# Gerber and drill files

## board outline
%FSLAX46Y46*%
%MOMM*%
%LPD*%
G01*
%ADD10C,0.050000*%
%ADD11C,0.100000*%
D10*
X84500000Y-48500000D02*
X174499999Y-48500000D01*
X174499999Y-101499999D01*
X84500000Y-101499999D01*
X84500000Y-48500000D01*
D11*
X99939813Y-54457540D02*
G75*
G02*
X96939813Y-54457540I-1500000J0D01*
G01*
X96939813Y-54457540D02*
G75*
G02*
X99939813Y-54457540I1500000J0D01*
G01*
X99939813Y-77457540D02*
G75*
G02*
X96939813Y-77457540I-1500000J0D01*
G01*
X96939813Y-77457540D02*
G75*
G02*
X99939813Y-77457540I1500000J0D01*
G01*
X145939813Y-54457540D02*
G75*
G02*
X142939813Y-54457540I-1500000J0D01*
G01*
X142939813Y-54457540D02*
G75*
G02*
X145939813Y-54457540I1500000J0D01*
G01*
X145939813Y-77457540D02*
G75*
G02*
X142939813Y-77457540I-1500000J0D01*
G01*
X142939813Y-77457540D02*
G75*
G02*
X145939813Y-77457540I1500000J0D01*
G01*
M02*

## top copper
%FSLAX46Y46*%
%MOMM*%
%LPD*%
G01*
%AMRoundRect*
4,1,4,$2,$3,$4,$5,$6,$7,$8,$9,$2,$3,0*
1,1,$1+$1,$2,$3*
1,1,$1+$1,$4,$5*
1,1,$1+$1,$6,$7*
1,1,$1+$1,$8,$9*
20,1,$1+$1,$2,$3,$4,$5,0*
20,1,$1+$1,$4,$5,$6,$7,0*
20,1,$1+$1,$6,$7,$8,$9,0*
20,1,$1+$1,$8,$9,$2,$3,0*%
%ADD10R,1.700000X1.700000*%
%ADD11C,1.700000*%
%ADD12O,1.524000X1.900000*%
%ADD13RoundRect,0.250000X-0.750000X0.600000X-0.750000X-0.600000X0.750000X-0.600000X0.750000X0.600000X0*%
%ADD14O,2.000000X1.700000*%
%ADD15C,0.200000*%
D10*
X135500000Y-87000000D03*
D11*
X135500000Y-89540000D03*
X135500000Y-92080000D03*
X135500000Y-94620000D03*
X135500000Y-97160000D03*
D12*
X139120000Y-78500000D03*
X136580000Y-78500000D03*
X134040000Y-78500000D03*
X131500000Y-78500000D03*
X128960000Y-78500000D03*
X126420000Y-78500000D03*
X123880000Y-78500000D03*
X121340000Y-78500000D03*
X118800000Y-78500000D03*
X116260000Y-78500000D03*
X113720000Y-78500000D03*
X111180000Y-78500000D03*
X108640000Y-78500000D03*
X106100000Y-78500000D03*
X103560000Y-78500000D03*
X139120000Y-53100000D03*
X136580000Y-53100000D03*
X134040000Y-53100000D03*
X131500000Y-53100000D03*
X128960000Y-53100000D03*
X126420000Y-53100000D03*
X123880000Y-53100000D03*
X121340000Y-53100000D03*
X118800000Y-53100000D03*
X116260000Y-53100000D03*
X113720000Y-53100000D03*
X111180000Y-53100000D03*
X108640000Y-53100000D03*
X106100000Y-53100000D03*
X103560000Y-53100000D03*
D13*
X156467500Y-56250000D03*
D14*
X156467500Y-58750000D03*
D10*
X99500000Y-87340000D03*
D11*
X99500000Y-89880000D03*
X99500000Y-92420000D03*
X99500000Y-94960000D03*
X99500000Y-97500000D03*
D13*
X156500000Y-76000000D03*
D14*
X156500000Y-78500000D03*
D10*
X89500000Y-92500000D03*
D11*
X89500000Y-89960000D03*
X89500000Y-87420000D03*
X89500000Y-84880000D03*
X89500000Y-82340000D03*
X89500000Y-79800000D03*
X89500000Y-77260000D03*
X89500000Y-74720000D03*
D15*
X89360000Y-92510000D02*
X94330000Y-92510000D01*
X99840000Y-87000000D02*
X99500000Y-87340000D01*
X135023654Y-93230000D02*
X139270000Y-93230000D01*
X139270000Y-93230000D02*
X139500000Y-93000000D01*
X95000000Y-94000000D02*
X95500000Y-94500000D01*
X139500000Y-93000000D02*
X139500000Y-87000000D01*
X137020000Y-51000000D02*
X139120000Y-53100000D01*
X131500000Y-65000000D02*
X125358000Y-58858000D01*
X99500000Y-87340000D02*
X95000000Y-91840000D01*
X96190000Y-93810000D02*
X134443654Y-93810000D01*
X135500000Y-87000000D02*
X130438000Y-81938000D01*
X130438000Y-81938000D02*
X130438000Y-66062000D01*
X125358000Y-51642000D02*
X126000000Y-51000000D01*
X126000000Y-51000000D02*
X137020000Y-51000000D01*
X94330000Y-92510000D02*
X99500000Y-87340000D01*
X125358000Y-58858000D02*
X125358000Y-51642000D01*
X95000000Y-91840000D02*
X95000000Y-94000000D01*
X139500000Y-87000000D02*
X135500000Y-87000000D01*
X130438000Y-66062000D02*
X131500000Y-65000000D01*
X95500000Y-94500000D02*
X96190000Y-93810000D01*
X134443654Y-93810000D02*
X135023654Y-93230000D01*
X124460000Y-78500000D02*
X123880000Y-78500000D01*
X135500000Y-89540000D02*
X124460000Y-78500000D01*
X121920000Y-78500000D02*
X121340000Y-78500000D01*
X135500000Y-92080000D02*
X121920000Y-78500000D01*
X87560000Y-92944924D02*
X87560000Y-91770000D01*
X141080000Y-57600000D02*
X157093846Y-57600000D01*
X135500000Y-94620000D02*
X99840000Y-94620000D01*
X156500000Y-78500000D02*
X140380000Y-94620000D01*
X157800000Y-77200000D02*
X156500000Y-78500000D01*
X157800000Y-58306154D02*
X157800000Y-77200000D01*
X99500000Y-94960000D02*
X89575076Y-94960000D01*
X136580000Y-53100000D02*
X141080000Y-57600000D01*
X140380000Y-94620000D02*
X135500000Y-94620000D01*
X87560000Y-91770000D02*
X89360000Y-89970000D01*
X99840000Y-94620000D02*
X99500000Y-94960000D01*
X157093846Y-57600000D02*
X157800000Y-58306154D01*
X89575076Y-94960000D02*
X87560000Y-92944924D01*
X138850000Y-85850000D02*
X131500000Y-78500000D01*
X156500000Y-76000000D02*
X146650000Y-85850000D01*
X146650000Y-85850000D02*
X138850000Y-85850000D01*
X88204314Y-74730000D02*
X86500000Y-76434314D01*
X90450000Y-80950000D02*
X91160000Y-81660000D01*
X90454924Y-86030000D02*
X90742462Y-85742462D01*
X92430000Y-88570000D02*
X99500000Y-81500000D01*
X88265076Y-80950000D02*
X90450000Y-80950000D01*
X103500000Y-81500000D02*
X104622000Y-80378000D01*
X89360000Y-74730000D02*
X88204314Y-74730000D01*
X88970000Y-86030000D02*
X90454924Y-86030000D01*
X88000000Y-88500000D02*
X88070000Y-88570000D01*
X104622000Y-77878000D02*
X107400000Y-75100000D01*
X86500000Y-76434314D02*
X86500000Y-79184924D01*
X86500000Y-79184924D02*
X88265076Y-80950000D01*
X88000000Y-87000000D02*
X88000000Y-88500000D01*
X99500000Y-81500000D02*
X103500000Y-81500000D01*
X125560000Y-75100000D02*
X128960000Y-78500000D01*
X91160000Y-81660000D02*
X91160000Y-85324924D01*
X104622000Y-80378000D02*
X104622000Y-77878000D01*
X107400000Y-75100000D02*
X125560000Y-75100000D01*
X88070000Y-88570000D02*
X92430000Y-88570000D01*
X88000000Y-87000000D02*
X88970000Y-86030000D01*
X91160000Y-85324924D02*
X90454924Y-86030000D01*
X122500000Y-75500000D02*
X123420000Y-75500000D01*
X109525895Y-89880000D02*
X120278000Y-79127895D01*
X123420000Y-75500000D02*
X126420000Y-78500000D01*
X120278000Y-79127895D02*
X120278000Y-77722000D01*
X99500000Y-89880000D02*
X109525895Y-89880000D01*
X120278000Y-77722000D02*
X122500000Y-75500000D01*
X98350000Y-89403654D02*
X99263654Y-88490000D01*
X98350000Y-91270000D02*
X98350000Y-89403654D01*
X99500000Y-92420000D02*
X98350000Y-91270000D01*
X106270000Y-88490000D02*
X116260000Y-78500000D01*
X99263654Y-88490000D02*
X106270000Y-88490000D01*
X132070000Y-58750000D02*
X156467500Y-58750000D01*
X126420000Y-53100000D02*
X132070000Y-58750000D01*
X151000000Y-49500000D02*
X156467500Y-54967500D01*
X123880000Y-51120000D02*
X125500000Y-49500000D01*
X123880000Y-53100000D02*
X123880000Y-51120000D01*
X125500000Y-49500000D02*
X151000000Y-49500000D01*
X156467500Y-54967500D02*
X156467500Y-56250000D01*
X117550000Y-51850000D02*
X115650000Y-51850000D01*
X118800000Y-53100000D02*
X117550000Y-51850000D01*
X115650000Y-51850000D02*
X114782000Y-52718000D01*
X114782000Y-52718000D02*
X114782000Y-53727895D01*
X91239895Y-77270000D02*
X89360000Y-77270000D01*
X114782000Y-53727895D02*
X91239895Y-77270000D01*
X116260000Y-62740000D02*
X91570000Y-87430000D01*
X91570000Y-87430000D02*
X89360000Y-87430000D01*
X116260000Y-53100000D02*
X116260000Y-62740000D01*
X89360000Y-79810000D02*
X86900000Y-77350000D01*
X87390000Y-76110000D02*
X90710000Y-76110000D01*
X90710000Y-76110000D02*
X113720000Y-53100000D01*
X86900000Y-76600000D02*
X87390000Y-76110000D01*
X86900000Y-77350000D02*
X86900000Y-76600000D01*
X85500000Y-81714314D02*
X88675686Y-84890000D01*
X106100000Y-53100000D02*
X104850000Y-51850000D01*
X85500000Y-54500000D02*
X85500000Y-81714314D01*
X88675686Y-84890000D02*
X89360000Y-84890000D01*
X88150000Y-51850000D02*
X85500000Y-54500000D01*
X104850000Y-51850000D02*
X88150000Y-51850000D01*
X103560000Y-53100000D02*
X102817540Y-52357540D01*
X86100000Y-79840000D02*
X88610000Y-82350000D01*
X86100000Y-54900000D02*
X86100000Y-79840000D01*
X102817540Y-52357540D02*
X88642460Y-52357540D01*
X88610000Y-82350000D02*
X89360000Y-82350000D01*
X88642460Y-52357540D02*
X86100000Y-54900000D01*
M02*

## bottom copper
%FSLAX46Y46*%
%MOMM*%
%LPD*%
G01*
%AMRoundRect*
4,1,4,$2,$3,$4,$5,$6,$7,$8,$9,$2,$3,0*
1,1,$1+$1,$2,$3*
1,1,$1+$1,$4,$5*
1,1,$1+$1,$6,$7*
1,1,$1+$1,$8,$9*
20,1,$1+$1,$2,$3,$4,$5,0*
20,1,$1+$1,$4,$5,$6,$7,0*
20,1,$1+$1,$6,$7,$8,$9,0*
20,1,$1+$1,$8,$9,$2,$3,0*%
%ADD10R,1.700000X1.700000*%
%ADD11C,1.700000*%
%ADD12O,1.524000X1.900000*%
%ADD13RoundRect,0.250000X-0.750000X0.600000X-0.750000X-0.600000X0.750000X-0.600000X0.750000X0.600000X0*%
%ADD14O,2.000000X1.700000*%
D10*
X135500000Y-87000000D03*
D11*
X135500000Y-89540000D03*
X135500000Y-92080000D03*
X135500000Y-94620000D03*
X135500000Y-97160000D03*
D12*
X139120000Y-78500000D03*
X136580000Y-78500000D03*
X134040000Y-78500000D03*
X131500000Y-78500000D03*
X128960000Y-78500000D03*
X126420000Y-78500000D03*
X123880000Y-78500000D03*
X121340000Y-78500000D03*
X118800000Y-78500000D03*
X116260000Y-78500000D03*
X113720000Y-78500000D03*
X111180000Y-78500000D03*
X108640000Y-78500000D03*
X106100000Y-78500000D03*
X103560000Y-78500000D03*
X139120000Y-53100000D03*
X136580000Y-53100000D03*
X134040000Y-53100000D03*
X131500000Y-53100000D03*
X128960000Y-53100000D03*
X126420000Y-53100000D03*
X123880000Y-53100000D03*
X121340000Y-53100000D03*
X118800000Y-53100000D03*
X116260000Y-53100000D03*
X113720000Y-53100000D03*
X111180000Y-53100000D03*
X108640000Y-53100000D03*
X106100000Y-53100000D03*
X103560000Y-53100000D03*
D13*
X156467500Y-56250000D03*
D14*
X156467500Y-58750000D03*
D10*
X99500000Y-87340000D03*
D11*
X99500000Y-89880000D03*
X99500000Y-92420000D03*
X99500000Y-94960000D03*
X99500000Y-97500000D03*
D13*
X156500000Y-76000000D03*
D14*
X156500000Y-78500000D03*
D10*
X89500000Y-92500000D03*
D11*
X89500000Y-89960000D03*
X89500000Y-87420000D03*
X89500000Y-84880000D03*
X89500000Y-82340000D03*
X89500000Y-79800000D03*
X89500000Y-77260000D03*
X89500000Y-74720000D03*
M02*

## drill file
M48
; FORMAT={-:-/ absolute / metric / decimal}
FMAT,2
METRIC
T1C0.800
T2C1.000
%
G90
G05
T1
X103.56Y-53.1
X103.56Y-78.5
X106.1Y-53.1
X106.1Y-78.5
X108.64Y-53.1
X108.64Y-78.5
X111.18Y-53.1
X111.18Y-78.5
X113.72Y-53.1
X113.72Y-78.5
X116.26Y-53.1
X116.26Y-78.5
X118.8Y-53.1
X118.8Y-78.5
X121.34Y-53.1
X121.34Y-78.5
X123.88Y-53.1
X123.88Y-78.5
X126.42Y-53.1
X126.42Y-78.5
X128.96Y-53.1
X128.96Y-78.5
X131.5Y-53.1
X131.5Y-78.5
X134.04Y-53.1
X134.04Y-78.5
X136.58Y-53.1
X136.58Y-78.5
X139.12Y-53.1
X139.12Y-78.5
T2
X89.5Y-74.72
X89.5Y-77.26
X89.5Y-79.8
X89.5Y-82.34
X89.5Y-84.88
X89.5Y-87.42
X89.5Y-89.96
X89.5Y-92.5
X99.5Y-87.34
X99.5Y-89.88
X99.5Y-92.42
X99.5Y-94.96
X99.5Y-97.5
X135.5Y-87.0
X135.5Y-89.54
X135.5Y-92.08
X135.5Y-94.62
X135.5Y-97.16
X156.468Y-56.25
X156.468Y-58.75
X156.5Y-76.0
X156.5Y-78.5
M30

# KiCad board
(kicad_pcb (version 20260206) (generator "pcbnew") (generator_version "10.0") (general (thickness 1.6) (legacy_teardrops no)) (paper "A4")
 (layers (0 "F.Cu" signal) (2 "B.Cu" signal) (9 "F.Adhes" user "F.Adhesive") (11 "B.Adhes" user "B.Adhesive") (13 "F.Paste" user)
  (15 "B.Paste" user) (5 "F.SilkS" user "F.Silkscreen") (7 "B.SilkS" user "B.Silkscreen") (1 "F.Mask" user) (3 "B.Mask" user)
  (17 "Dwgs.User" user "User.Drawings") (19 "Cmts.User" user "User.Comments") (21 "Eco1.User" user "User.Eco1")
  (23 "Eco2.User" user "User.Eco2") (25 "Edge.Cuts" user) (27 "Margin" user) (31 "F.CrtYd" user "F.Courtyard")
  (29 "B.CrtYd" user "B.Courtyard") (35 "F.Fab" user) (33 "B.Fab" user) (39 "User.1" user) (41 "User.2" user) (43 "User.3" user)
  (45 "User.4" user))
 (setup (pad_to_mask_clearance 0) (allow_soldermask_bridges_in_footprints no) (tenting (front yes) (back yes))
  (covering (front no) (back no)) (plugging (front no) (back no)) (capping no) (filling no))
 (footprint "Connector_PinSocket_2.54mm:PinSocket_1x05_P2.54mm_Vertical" (layer "F.Cu") (at 135.5 87)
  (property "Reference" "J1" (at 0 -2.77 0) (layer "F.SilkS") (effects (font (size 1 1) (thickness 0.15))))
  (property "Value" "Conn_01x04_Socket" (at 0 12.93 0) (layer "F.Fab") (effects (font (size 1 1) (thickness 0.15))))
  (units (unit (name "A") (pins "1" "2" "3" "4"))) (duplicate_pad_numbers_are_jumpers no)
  (pad "1" thru_hole rect (at 0 0) (size 1.7 1.7) (drill 1) (layers "*.Cu" "*.Mask") (remove_unused_layers no) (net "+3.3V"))
  (pad "2" thru_hole circle (at 0 2.54) (size 1.7 1.7) (drill 1) (layers "*.Cu" "*.Mask") (remove_unused_layers no) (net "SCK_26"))
  (pad "3" thru_hole circle (at 0 5.08) (size 1.7 1.7) (drill 1) (layers "*.Cu" "*.Mask") (remove_unused_layers no) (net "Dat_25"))
  (pad "4" thru_hole circle (at 0 7.62) (size 1.7 1.7) (drill 1) (layers "*.Cu" "*.Mask") (remove_unused_layers no) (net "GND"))
  (pad "5" thru_hole circle (at 0 10.16) (size 1.7 1.7) (drill 1) (layers "*.Cu" "*.Mask") (remove_unused_layers no)))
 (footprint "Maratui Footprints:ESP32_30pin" (layer "F.Cu") (at 121.579813 66.02754 180)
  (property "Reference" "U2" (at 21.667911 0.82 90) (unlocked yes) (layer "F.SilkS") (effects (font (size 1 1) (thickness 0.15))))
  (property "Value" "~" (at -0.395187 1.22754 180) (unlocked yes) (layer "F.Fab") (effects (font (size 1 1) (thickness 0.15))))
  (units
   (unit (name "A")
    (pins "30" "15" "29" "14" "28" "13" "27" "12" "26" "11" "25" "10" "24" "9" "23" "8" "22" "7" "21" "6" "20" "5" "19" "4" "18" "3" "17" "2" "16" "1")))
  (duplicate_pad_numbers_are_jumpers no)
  (fp_circle (center 23.14 11.57) (end 24.64 11.57) (stroke (width 0.1) (type default)) (fill no) (layer "Edge.Cuts"))
  (fp_circle (center 23.14 -11.43) (end 24.64 -11.43) (stroke (width 0.1) (type default)) (fill no) (layer "Edge.Cuts"))
  (fp_circle (center -22.86 11.57) (end -21.36 11.57) (stroke (width 0.1) (type default)) (fill no) (layer "Edge.Cuts"))
  (fp_circle (center -22.86 -11.43) (end -21.36 -11.43) (stroke (width 0.1) (type default)) (fill no) (layer "Edge.Cuts"))
  (pad "1" thru_hole oval (at -17.540187 -12.47246 180) (size 1.524 1.9) (drill 0.8) (layers "*.Cu" "*.Mask") (remove_unused_layers no)
   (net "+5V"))
  (pad "2" thru_hole oval (at -15.000187 -12.47246 180) (size 1.524 1.9) (drill 0.8) (layers "*.Cu" "*.Mask") (remove_unused_layers no)
   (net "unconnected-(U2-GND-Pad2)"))
  (pad "3" thru_hole oval (at -12.460187 -12.47246 180) (size 1.524 1.9) (drill 0.8) (layers "*.Cu" "*.Mask") (remove_unused_layers no)
   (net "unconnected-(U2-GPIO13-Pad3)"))
  (pad "4" thru_hole oval (at -9.920187 -12.47246 180) (size 1.524 1.9) (drill 0.8) (layers "*.Cu" "*.Mask") (remove_unused_layers no)
   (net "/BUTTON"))
  (pad "5" thru_hole oval (at -7.380187 -12.47246 180) (size 1.524 1.9) (drill 0.8) (layers "*.Cu" "*.Mask") (remove_unused_layers no)
   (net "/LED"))
  (pad "6" thru_hole oval (at -4.840187 -12.47246 180) (size 1.524 1.9) (drill 0.8) (layers "*.Cu" "*.Mask") (remove_unused_layers no)
   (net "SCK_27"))
  (pad "7" thru_hole oval (at -2.300187 -12.47246 180) (size 1.524 1.9) (drill 0.8) (layers "*.Cu" "*.Mask") (remove_unused_layers no)
   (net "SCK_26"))
  (pad "8" thru_hole oval (at 0.239813 -12.47246 180) (size 1.524 1.9) (drill 0.8) (layers "*.Cu" "*.Mask") (remove_unused_layers no)
   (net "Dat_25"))
  (pad "9" thru_hole oval (at 2.779813 -12.47246 180) (size 1.524 1.9) (drill 0.8) (layers "*.Cu" "*.Mask") (remove_unused_layers no)
   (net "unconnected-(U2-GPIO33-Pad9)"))
  (pad "10" thru_hole oval (at 5.319813 -12.47246 180) (size 1.524 1.9) (drill 0.8) (layers "*.Cu" "*.Mask") (remove_unused_layers no)
   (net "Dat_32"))
  (pad "11" thru_hole oval (at 7.859813 -12.47246 180) (size 1.524 1.9) (drill 0.8) (layers "*.Cu" "*.Mask") (remove_unused_layers no)
   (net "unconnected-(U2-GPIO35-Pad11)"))
  (pad "12" thru_hole oval (at 10.399813 -12.47246 180) (size 1.524 1.9) (drill 0.8) (layers "*.Cu" "*.Mask") (remove_unused_layers no)
   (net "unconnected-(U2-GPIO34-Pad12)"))
  (pad "13" thru_hole oval (at 12.939813 -12.47246 180) (size 1.524 1.9) (drill 0.8) (layers "*.Cu" "*.Mask") (remove_unused_layers no)
   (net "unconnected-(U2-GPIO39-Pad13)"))
  (pad "14" thru_hole oval (at 15.479813 -12.47246 180) (size 1.524 1.9) (drill 0.8) (layers "*.Cu" "*.Mask") (remove_unused_layers no)
   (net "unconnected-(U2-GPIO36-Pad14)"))
  (pad "15" thru_hole oval (at 18.019813 -12.47246 180) (size 1.524 1.9) (drill 0.8) (layers "*.Cu" "*.Mask") (remove_unused_layers no)
   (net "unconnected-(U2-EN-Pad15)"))
  (pad "16" thru_hole oval (at -17.540187 12.92754 180) (size 1.524 1.9) (drill 0.8) (layers "*.Cu" "*.Mask") (remove_unused_layers no)
   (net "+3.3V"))
  (pad "17" thru_hole oval (at -15.000187 12.92754 180) (size 1.524 1.9) (drill 0.8) (layers "*.Cu" "*.Mask") (remove_unused_layers no)
   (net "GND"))
  (pad "18" thru_hole oval (at -12.460187 12.92754 180) (size 1.524 1.9) (drill 0.8) (layers "*.Cu" "*.Mask") (remove_unused_layers no)
   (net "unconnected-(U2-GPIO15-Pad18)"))
  (pad "19" thru_hole oval (at -9.920187 12.92754 180) (size 1.524 1.9) (drill 0.8) (layers "*.Cu" "*.Mask") (remove_unused_layers no)
   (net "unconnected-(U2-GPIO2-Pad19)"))
  (pad "20" thru_hole oval (at -7.380187 12.92754 180) (size 1.524 1.9) (drill 0.8) (layers "*.Cu" "*.Mask") (remove_unused_layers no)
   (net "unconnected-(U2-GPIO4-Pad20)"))
  (pad "21" thru_hole oval (at -4.840187 12.92754 180) (size 1.524 1.9) (drill 0.8) (layers "*.Cu" "*.Mask") (remove_unused_layers no)
   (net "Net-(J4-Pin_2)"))
  (pad "22" thru_hole oval (at -2.300187 12.92754 180) (size 1.524 1.9) (drill 0.8) (layers "*.Cu" "*.Mask") (remove_unused_layers no)
   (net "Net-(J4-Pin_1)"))
  (pad "23" thru_hole oval (at 0.239813 12.92754 180) (size 1.524 1.9) (drill 0.8) (layers "*.Cu" "*.Mask") (remove_unused_layers no)
   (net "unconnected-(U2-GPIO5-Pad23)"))
  (pad "24" thru_hole oval (at 2.779813 12.92754 180) (size 1.524 1.9) (drill 0.8) (layers "*.Cu" "*.Mask") (remove_unused_layers no)
   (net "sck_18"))
  (pad "25" thru_hole oval (at 5.319813 12.92754 180) (size 1.524 1.9) (drill 0.8) (layers "*.Cu" "*.Mask") (remove_unused_layers no)
   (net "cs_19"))
  (pad "26" thru_hole oval (at 7.859813 12.92754 180) (size 1.524 1.9) (drill 0.8) (layers "*.Cu" "*.Mask") (remove_unused_layers no)
   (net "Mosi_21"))
  (pad "27" thru_hole oval (at 10.399813 12.92754 180) (size 1.524 1.9) (drill 0.8) (layers "*.Cu" "*.Mask") (remove_unused_layers no)
   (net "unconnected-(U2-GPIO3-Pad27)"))
  (pad "28" thru_hole oval (at 12.939813 12.92754 180) (size 1.524 1.9) (drill 0.8) (layers "*.Cu" "*.Mask") (remove_unused_layers no)
   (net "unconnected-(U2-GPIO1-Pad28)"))
  (pad "29" thru_hole oval (at 15.479813 12.92754 180) (size 1.524 1.9) (drill 0.8) (layers "*.Cu" "*.Mask") (remove_unused_layers no)
   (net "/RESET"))
  (pad "30" thru_hole oval (at 18.019813 12.92754 180) (size 1.524 1.9) (drill 0.8) (layers "*.Cu" "*.Mask") (remove_unused_layers no)
   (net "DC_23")))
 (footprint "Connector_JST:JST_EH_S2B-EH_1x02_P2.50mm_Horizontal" (layer "F.Cu") (at 156.4675 56.25 -90)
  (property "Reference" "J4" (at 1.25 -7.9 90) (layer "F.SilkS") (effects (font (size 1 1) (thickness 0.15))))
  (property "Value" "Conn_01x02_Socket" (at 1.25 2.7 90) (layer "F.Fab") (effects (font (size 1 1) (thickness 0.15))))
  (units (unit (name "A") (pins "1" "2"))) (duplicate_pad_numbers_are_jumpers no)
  (pad "1" thru_hole roundrect (at 0 0 270) (size 1.7 2) (drill 1) (layers "*.Cu" "*.Mask") (remove_unused_layers no)
   (roundrect_rratio 0.147059) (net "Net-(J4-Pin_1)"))
  (pad "2" thru_hole oval (at 2.5 0 270) (size 1.7 2) (drill 1) (layers "*.Cu" "*.Mask") (remove_unused_layers no) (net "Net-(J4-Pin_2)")))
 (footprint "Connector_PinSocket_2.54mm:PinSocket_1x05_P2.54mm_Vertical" (layer "F.Cu") (at 99.5 87.34)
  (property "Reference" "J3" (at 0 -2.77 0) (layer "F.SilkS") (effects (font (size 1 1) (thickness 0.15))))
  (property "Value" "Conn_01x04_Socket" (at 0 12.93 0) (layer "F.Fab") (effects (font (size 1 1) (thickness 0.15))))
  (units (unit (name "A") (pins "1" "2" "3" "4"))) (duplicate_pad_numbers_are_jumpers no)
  (pad "1" thru_hole rect (at 0 0) (size 1.7 1.7) (drill 1) (layers "*.Cu" "*.Mask") (remove_unused_layers no) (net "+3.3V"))
  (pad "2" thru_hole circle (at 0 2.54) (size 1.7 1.7) (drill 1) (layers "*.Cu" "*.Mask") (remove_unused_layers no) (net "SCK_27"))
  (pad "3" thru_hole circle (at 0 5.08) (size 1.7 1.7) (drill 1) (layers "*.Cu" "*.Mask") (remove_unused_layers no) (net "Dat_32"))
  (pad "4" thru_hole circle (at 0 7.62) (size 1.7 1.7) (drill 1) (layers "*.Cu" "*.Mask") (remove_unused_layers no) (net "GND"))
  (pad "5" thru_hole circle (at 0 10.16) (size 1.7 1.7) (drill 1) (layers "*.Cu" "*.Mask") (remove_unused_layers no)))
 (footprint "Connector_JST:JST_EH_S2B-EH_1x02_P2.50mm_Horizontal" (layer "F.Cu") (at 156.5 76 -90)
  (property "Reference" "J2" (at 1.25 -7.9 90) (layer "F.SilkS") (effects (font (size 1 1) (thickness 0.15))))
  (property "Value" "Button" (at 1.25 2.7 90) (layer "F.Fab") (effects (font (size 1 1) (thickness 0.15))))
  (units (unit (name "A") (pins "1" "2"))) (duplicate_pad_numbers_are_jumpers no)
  (pad "1" thru_hole roundrect (at 0 0 270) (size 1.7 2) (drill 1) (layers "*.Cu" "*.Mask") (remove_unused_layers no)
   (roundrect_rratio 0.147059) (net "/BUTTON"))
  (pad "2" thru_hole oval (at 2.5 0 270) (size 1.7 2) (drill 1) (layers "*.Cu" "*.Mask") (remove_unused_layers no) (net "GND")))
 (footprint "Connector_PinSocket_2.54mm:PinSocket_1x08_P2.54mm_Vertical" (layer "F.Cu") (at 89.5 92.5 180)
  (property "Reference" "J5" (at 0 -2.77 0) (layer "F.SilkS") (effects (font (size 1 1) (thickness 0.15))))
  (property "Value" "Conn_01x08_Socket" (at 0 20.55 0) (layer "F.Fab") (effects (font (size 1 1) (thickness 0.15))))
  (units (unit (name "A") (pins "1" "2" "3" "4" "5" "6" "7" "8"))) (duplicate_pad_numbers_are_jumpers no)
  (pad "1" thru_hole rect (at 0 0 180) (size 1.7 1.7) (drill 1) (layers "*.Cu" "*.Mask") (remove_unused_layers no) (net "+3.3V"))
  (pad "2" thru_hole circle (at 0 2.54 180) (size 1.7 1.7) (drill 1) (layers "*.Cu" "*.Mask") (remove_unused_layers no) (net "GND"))
  (pad "3" thru_hole circle (at 0 5.08 180) (size 1.7 1.7) (drill 1) (layers "*.Cu" "*.Mask") (remove_unused_layers no) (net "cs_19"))
  (pad "4" thru_hole circle (at 0 7.62 180) (size 1.7 1.7) (drill 1) (layers "*.Cu" "*.Mask") (remove_unused_layers no) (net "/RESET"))
  (pad "5" thru_hole circle (at 0 10.16 180) (size 1.7 1.7) (drill 1) (layers "*.Cu" "*.Mask") (remove_unused_layers no) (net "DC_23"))
  (pad "6" thru_hole circle (at 0 12.7 180) (size 1.7 1.7) (drill 1) (layers "*.Cu" "*.Mask") (remove_unused_layers no) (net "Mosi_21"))
  (pad "7" thru_hole circle (at 0 15.24 180) (size 1.7 1.7) (drill 1) (layers "*.Cu" "*.Mask") (remove_unused_layers no) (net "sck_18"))
  (pad "8" thru_hole circle (at 0 17.78 180) (size 1.7 1.7) (drill 1) (layers "*.Cu" "*.Mask") (remove_unused_layers no) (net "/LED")))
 (gr_rect (start 84.5 48.5) (end 174.499999 101.499999) (stroke (width 0.05) (type default)) (fill no) (layer "Edge.Cuts"))
 (segment (start 89.36 92.51) (end 94.33 92.51) (width 0.2) (layer "F.Cu") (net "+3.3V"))
 (segment (start 99.84 87) (end 99.5 87.34) (width 0.2) (layer "F.Cu") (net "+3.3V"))
 (segment (start 135.023654 93.23) (end 139.27 93.23) (width 0.2) (layer "F.Cu") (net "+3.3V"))
 (segment (start 139.27 93.23) (end 139.5 93) (width 0.2) (layer "F.Cu") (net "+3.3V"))
 (segment (start 95 94) (end 95.5 94.5) (width 0.2) (layer "F.Cu") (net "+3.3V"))
 (segment (start 139.5 93) (end 139.5 87) (width 0.2) (layer "F.Cu") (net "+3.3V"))
 (segment (start 137.02 51) (end 139.12 53.1) (width 0.2) (layer "F.Cu") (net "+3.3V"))
 (segment (start 131.5 65) (end 125.358 58.858) (width 0.2) (layer "F.Cu") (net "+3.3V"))
 (segment (start 99.5 87.34) (end 95 91.84) (width 0.2) (layer "F.Cu") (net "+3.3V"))
 (segment (start 96.19 93.81) (end 134.443654 93.81) (width 0.2) (layer "F.Cu") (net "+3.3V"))
 (segment (start 135.5 87) (end 130.438 81.938) (width 0.2) (layer "F.Cu") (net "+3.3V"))
 (segment (start 130.438 81.938) (end 130.438 66.062) (width 0.2) (layer "F.Cu") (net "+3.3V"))
 (segment (start 125.358 51.642) (end 126 51) (width 0.2) (layer "F.Cu") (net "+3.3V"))
 (segment (start 126 51) (end 137.02 51) (width 0.2) (layer "F.Cu") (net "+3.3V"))
 (segment (start 94.33 92.51) (end 99.5 87.34) (width 0.2) (layer "F.Cu") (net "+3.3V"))
 (segment (start 125.358 58.858) (end 125.358 51.642) (width 0.2) (layer "F.Cu") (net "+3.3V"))
 (segment (start 95 91.84) (end 95 94) (width 0.2) (layer "F.Cu") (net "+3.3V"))
 (segment (start 139.5 87) (end 135.5 87) (width 0.2) (layer "F.Cu") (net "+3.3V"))
 (segment (start 130.438 66.062) (end 131.5 65) (width 0.2) (layer "F.Cu") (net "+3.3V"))
 (segment (start 95.5 94.5) (end 96.19 93.81) (width 0.2) (layer "F.Cu") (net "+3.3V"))
 (segment (start 134.443654 93.81) (end 135.023654 93.23) (width 0.2) (layer "F.Cu") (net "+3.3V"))
 (segment (start 124.46 78.5) (end 123.88 78.5) (width 0.2) (layer "F.Cu") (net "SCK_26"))
 (segment (start 135.5 89.54) (end 124.46 78.5) (width 0.2) (layer "F.Cu") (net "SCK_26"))
 (segment (start 121.92 78.5) (end 121.34 78.5) (width 0.2) (layer "F.Cu") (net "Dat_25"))
 (segment (start 135.5 92.08) (end 121.92 78.5) (width 0.2) (layer "F.Cu") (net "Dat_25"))
 (segment (start 87.56 92.944924) (end 87.56 91.77) (width 0.2) (layer "F.Cu") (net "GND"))
 (segment (start 141.08 57.6) (end 157.093846 57.6) (width 0.2) (layer "F.Cu") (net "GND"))
 (segment (start 135.5 94.62) (end 99.84 94.62) (width 0.2) (layer "F.Cu") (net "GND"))
 (segment (start 156.5 78.5) (end 140.38 94.62) (width 0.2) (layer "F.Cu") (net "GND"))
 (segment (start 157.8 77.2) (end 156.5 78.5) (width 0.2) (layer "F.Cu") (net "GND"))
 (segment (start 157.8 58.306154) (end 157.8 77.2) (width 0.2) (layer "F.Cu") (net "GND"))
 (segment (start 99.5 94.96) (end 89.575076 94.96) (width 0.2) (layer "F.Cu") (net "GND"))
 (segment (start 136.58 53.1) (end 141.08 57.6) (width 0.2) (layer "F.Cu") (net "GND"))
 (segment (start 140.38 94.62) (end 135.5 94.62) (width 0.2) (layer "F.Cu") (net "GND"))
 (segment (start 87.56 91.77) (end 89.36 89.97) (width 0.2) (layer "F.Cu") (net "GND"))
 (segment (start 99.84 94.62) (end 99.5 94.96) (width 0.2) (layer "F.Cu") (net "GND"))
 (segment (start 157.093846 57.6) (end 157.8 58.306154) (width 0.2) (layer "F.Cu") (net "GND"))
 (segment (start 89.575076 94.96) (end 87.56 92.944924) (width 0.2) (layer "F.Cu") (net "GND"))
 (segment (start 138.85 85.85) (end 131.5 78.5) (width 0.2) (layer "F.Cu") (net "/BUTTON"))
 (segment (start 156.5 76) (end 146.65 85.85) (width 0.2) (layer "F.Cu") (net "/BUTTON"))
 (segment (start 146.65 85.85) (end 138.85 85.85) (width 0.2) (layer "F.Cu") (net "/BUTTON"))
 (segment (start 88.204314 74.73) (end 86.5 76.434314) (width 0.2) (layer "F.Cu") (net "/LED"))
 (segment (start 90.45 80.95) (end 91.16 81.66) (width 0.2) (layer "F.Cu") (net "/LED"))
 (segment (start 90.454924 86.03) (end 90.742462 85.742462) (width 0.2) (layer "F.Cu") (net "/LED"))
 (segment (start 92.43 88.57) (end 99.5 81.5) (width 0.2) (layer "F.Cu") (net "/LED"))
 (segment (start 88.265076 80.95) (end 90.45 80.95) (width 0.2) (layer "F.Cu") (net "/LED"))
 (segment (start 103.5 81.5) (end 104.622 80.378) (width 0.2) (layer "F.Cu") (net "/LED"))
 (segment (start 89.36 74.73) (end 88.204314 74.73) (width 0.2) (layer "F.Cu") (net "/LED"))
 (segment (start 88.97 86.03) (end 90.454924 86.03) (width 0.2) (layer "F.Cu") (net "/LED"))
 (segment (start 88 88.5) (end 88.07 88.57) (width 0.2) (layer "F.Cu") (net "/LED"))
 (segment (start 104.622 77.878) (end 107.4 75.1) (width 0.2) (layer "F.Cu") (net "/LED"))
 (segment (start 86.5 76.434314) (end 86.5 79.184924) (width 0.2) (layer "F.Cu") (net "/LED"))
 (segment (start 86.5 79.184924) (end 88.265076 80.95) (width 0.2) (layer "F.Cu") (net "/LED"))
 (segment (start 88 87) (end 88 88.5) (width 0.2) (layer "F.Cu") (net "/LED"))
 (segment (start 99.5 81.5) (end 103.5 81.5) (width 0.2) (layer "F.Cu") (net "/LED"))
 (segment (start 125.56 75.1) (end 128.96 78.5) (width 0.2) (layer "F.Cu") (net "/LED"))
 (segment (start 91.16 81.66) (end 91.16 85.324924) (width 0.2) (layer "F.Cu") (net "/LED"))
 (segment (start 104.622 80.378) (end 104.622 77.878) (width 0.2) (layer "F.Cu") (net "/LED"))
 (segment (start 107.4 75.1) (end 125.56 75.1) (width 0.2) (layer "F.Cu") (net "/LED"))
 (segment (start 88.07 88.57) (end 92.43 88.57) (width 0.2) (layer "F.Cu") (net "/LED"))
 (segment (start 88 87) (end 88.97 86.03) (width 0.2) (layer "F.Cu") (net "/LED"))
 (segment (start 91.16 85.324924) (end 90.454924 86.03) (width 0.2) (layer "F.Cu") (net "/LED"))
 (segment (start 122.5 75.5) (end 123.42 75.5) (width 0.2) (layer "F.Cu") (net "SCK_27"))
 (segment (start 109.525895 89.88) (end 120.278 79.127895) (width 0.2) (layer "F.Cu") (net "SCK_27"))
 (segment (start 123.42 75.5) (end 126.42 78.5) (width 0.2) (layer "F.Cu") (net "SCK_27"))
 (segment (start 120.278 79.127895) (end 120.278 77.722) (width 0.2) (layer "F.Cu") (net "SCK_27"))
 (segment (start 99.5 89.88) (end 109.525895 89.88) (width 0.2) (layer "F.Cu") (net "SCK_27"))
 (segment (start 120.278 77.722) (end 122.5 75.5) (width 0.2) (layer "F.Cu") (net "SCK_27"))
 (segment (start 98.35 89.403654) (end 99.263654 88.49) (width 0.2) (layer "F.Cu") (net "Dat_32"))
 (segment (start 98.35 91.27) (end 98.35 89.403654) (width 0.2) (layer "F.Cu") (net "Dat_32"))
 (segment (start 99.5 92.42) (end 98.35 91.27) (width 0.2) (layer "F.Cu") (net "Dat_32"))
 (segment (start 106.27 88.49) (end 116.26 78.5) (width 0.2) (layer "F.Cu") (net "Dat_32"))
 (segment (start 99.263654 88.49) (end 106.27 88.49) (width 0.2) (layer "F.Cu") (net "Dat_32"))
 (segment (start 132.07 58.75) (end 156.4675 58.75) (width 0.2) (layer "F.Cu") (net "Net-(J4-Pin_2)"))
 (segment (start 126.42 53.1) (end 132.07 58.75) (width 0.2) (layer "F.Cu") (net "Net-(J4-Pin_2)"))
 (segment (start 151 49.5) (end 156.4675 54.9675) (width 0.2) (layer "F.Cu") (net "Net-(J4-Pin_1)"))
 (segment (start 123.88 51.12) (end 125.5 49.5) (width 0.2) (layer "F.Cu") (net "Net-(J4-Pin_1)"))
 (segment (start 123.88 53.1) (end 123.88 51.12) (width 0.2) (layer "F.Cu") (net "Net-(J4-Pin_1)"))
 (segment (start 125.5 49.5) (end 151 49.5) (width 0.2) (layer "F.Cu") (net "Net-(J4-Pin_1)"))
 (segment (start 156.4675 54.9675) (end 156.4675 56.25) (width 0.2) (layer "F.Cu") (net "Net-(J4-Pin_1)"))
 (segment (start 117.55 51.85) (end 115.65 51.85) (width 0.2) (layer "F.Cu") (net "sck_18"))
 (segment (start 118.8 53.1) (end 117.55 51.85) (width 0.2) (layer "F.Cu") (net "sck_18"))
 (segment (start 115.65 51.85) (end 114.782 52.718) (width 0.2) (layer "F.Cu") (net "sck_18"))
 (segment (start 114.782 52.718) (end 114.782 53.727895) (width 0.2) (layer "F.Cu") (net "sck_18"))
 (segment (start 91.239895 77.27) (end 89.36 77.27) (width 0.2) (layer "F.Cu") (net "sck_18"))
 (segment (start 114.782 53.727895) (end 91.239895 77.27) (width 0.2) (layer "F.Cu") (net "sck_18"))
 (segment (start 116.26 62.74) (end 91.57 87.43) (width 0.2) (layer "F.Cu") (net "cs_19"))
 (segment (start 91.57 87.43) (end 89.36 87.43) (width 0.2) (layer "F.Cu") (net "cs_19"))
 (segment (start 116.26 53.1) (end 116.26 62.74) (width 0.2) (layer "F.Cu") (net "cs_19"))
 (segment (start 89.36 79.81) (end 86.9 77.35) (width 0.2) (layer "F.Cu") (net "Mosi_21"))
 (segment (start 87.39 76.11) (end 90.71 76.11) (width 0.2) (layer "F.Cu") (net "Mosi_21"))
 (segment (start 90.71 76.11) (end 113.72 53.1) (width 0.2) (layer "F.Cu") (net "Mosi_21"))
 (segment (start 86.9 76.6) (end 87.39 76.11) (width 0.2) (layer "F.Cu") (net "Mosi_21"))
 (segment (start 86.9 77.35) (end 86.9 76.6) (width 0.2) (layer "F.Cu") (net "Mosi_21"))
 (segment (start 85.5 81.714314) (end 88.675686 84.89) (width 0.2) (layer "F.Cu") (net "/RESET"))
 (segment (start 106.1 53.1) (end 104.85 51.85) (width 0.2) (layer "F.Cu") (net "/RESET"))
 (segment (start 85.5 54.5) (end 85.5 81.714314) (width 0.2) (layer "F.Cu") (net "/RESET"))
 (segment (start 88.675686 84.89) (end 89.36 84.89) (width 0.2) (layer "F.Cu") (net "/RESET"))
 (segment (start 88.15 51.85) (end 85.5 54.5) (width 0.2) (layer "F.Cu") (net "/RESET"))
 (segment (start 104.85 51.85) (end 88.15 51.85) (width 0.2) (layer "F.Cu") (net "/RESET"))
 (segment (start 103.56 53.1) (end 102.81754 52.35754) (width 0.2) (layer "F.Cu") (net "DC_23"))
 (segment (start 86.1 79.84) (end 88.61 82.35) (width 0.2) (layer "F.Cu") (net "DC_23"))
 (segment (start 86.1 54.9) (end 86.1 79.84) (width 0.2) (layer "F.Cu") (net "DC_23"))
 (segment (start 102.81754 52.35754) (end 88.64246 52.35754) (width 0.2) (layer "F.Cu") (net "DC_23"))
 (segment (start 88.61 82.35) (end 89.36 82.35) (width 0.2) (layer "F.Cu") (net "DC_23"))
 (segment (start 88.64246 52.35754) (end 86.1 54.9) (width 0.2) (layer "F.Cu") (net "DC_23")))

